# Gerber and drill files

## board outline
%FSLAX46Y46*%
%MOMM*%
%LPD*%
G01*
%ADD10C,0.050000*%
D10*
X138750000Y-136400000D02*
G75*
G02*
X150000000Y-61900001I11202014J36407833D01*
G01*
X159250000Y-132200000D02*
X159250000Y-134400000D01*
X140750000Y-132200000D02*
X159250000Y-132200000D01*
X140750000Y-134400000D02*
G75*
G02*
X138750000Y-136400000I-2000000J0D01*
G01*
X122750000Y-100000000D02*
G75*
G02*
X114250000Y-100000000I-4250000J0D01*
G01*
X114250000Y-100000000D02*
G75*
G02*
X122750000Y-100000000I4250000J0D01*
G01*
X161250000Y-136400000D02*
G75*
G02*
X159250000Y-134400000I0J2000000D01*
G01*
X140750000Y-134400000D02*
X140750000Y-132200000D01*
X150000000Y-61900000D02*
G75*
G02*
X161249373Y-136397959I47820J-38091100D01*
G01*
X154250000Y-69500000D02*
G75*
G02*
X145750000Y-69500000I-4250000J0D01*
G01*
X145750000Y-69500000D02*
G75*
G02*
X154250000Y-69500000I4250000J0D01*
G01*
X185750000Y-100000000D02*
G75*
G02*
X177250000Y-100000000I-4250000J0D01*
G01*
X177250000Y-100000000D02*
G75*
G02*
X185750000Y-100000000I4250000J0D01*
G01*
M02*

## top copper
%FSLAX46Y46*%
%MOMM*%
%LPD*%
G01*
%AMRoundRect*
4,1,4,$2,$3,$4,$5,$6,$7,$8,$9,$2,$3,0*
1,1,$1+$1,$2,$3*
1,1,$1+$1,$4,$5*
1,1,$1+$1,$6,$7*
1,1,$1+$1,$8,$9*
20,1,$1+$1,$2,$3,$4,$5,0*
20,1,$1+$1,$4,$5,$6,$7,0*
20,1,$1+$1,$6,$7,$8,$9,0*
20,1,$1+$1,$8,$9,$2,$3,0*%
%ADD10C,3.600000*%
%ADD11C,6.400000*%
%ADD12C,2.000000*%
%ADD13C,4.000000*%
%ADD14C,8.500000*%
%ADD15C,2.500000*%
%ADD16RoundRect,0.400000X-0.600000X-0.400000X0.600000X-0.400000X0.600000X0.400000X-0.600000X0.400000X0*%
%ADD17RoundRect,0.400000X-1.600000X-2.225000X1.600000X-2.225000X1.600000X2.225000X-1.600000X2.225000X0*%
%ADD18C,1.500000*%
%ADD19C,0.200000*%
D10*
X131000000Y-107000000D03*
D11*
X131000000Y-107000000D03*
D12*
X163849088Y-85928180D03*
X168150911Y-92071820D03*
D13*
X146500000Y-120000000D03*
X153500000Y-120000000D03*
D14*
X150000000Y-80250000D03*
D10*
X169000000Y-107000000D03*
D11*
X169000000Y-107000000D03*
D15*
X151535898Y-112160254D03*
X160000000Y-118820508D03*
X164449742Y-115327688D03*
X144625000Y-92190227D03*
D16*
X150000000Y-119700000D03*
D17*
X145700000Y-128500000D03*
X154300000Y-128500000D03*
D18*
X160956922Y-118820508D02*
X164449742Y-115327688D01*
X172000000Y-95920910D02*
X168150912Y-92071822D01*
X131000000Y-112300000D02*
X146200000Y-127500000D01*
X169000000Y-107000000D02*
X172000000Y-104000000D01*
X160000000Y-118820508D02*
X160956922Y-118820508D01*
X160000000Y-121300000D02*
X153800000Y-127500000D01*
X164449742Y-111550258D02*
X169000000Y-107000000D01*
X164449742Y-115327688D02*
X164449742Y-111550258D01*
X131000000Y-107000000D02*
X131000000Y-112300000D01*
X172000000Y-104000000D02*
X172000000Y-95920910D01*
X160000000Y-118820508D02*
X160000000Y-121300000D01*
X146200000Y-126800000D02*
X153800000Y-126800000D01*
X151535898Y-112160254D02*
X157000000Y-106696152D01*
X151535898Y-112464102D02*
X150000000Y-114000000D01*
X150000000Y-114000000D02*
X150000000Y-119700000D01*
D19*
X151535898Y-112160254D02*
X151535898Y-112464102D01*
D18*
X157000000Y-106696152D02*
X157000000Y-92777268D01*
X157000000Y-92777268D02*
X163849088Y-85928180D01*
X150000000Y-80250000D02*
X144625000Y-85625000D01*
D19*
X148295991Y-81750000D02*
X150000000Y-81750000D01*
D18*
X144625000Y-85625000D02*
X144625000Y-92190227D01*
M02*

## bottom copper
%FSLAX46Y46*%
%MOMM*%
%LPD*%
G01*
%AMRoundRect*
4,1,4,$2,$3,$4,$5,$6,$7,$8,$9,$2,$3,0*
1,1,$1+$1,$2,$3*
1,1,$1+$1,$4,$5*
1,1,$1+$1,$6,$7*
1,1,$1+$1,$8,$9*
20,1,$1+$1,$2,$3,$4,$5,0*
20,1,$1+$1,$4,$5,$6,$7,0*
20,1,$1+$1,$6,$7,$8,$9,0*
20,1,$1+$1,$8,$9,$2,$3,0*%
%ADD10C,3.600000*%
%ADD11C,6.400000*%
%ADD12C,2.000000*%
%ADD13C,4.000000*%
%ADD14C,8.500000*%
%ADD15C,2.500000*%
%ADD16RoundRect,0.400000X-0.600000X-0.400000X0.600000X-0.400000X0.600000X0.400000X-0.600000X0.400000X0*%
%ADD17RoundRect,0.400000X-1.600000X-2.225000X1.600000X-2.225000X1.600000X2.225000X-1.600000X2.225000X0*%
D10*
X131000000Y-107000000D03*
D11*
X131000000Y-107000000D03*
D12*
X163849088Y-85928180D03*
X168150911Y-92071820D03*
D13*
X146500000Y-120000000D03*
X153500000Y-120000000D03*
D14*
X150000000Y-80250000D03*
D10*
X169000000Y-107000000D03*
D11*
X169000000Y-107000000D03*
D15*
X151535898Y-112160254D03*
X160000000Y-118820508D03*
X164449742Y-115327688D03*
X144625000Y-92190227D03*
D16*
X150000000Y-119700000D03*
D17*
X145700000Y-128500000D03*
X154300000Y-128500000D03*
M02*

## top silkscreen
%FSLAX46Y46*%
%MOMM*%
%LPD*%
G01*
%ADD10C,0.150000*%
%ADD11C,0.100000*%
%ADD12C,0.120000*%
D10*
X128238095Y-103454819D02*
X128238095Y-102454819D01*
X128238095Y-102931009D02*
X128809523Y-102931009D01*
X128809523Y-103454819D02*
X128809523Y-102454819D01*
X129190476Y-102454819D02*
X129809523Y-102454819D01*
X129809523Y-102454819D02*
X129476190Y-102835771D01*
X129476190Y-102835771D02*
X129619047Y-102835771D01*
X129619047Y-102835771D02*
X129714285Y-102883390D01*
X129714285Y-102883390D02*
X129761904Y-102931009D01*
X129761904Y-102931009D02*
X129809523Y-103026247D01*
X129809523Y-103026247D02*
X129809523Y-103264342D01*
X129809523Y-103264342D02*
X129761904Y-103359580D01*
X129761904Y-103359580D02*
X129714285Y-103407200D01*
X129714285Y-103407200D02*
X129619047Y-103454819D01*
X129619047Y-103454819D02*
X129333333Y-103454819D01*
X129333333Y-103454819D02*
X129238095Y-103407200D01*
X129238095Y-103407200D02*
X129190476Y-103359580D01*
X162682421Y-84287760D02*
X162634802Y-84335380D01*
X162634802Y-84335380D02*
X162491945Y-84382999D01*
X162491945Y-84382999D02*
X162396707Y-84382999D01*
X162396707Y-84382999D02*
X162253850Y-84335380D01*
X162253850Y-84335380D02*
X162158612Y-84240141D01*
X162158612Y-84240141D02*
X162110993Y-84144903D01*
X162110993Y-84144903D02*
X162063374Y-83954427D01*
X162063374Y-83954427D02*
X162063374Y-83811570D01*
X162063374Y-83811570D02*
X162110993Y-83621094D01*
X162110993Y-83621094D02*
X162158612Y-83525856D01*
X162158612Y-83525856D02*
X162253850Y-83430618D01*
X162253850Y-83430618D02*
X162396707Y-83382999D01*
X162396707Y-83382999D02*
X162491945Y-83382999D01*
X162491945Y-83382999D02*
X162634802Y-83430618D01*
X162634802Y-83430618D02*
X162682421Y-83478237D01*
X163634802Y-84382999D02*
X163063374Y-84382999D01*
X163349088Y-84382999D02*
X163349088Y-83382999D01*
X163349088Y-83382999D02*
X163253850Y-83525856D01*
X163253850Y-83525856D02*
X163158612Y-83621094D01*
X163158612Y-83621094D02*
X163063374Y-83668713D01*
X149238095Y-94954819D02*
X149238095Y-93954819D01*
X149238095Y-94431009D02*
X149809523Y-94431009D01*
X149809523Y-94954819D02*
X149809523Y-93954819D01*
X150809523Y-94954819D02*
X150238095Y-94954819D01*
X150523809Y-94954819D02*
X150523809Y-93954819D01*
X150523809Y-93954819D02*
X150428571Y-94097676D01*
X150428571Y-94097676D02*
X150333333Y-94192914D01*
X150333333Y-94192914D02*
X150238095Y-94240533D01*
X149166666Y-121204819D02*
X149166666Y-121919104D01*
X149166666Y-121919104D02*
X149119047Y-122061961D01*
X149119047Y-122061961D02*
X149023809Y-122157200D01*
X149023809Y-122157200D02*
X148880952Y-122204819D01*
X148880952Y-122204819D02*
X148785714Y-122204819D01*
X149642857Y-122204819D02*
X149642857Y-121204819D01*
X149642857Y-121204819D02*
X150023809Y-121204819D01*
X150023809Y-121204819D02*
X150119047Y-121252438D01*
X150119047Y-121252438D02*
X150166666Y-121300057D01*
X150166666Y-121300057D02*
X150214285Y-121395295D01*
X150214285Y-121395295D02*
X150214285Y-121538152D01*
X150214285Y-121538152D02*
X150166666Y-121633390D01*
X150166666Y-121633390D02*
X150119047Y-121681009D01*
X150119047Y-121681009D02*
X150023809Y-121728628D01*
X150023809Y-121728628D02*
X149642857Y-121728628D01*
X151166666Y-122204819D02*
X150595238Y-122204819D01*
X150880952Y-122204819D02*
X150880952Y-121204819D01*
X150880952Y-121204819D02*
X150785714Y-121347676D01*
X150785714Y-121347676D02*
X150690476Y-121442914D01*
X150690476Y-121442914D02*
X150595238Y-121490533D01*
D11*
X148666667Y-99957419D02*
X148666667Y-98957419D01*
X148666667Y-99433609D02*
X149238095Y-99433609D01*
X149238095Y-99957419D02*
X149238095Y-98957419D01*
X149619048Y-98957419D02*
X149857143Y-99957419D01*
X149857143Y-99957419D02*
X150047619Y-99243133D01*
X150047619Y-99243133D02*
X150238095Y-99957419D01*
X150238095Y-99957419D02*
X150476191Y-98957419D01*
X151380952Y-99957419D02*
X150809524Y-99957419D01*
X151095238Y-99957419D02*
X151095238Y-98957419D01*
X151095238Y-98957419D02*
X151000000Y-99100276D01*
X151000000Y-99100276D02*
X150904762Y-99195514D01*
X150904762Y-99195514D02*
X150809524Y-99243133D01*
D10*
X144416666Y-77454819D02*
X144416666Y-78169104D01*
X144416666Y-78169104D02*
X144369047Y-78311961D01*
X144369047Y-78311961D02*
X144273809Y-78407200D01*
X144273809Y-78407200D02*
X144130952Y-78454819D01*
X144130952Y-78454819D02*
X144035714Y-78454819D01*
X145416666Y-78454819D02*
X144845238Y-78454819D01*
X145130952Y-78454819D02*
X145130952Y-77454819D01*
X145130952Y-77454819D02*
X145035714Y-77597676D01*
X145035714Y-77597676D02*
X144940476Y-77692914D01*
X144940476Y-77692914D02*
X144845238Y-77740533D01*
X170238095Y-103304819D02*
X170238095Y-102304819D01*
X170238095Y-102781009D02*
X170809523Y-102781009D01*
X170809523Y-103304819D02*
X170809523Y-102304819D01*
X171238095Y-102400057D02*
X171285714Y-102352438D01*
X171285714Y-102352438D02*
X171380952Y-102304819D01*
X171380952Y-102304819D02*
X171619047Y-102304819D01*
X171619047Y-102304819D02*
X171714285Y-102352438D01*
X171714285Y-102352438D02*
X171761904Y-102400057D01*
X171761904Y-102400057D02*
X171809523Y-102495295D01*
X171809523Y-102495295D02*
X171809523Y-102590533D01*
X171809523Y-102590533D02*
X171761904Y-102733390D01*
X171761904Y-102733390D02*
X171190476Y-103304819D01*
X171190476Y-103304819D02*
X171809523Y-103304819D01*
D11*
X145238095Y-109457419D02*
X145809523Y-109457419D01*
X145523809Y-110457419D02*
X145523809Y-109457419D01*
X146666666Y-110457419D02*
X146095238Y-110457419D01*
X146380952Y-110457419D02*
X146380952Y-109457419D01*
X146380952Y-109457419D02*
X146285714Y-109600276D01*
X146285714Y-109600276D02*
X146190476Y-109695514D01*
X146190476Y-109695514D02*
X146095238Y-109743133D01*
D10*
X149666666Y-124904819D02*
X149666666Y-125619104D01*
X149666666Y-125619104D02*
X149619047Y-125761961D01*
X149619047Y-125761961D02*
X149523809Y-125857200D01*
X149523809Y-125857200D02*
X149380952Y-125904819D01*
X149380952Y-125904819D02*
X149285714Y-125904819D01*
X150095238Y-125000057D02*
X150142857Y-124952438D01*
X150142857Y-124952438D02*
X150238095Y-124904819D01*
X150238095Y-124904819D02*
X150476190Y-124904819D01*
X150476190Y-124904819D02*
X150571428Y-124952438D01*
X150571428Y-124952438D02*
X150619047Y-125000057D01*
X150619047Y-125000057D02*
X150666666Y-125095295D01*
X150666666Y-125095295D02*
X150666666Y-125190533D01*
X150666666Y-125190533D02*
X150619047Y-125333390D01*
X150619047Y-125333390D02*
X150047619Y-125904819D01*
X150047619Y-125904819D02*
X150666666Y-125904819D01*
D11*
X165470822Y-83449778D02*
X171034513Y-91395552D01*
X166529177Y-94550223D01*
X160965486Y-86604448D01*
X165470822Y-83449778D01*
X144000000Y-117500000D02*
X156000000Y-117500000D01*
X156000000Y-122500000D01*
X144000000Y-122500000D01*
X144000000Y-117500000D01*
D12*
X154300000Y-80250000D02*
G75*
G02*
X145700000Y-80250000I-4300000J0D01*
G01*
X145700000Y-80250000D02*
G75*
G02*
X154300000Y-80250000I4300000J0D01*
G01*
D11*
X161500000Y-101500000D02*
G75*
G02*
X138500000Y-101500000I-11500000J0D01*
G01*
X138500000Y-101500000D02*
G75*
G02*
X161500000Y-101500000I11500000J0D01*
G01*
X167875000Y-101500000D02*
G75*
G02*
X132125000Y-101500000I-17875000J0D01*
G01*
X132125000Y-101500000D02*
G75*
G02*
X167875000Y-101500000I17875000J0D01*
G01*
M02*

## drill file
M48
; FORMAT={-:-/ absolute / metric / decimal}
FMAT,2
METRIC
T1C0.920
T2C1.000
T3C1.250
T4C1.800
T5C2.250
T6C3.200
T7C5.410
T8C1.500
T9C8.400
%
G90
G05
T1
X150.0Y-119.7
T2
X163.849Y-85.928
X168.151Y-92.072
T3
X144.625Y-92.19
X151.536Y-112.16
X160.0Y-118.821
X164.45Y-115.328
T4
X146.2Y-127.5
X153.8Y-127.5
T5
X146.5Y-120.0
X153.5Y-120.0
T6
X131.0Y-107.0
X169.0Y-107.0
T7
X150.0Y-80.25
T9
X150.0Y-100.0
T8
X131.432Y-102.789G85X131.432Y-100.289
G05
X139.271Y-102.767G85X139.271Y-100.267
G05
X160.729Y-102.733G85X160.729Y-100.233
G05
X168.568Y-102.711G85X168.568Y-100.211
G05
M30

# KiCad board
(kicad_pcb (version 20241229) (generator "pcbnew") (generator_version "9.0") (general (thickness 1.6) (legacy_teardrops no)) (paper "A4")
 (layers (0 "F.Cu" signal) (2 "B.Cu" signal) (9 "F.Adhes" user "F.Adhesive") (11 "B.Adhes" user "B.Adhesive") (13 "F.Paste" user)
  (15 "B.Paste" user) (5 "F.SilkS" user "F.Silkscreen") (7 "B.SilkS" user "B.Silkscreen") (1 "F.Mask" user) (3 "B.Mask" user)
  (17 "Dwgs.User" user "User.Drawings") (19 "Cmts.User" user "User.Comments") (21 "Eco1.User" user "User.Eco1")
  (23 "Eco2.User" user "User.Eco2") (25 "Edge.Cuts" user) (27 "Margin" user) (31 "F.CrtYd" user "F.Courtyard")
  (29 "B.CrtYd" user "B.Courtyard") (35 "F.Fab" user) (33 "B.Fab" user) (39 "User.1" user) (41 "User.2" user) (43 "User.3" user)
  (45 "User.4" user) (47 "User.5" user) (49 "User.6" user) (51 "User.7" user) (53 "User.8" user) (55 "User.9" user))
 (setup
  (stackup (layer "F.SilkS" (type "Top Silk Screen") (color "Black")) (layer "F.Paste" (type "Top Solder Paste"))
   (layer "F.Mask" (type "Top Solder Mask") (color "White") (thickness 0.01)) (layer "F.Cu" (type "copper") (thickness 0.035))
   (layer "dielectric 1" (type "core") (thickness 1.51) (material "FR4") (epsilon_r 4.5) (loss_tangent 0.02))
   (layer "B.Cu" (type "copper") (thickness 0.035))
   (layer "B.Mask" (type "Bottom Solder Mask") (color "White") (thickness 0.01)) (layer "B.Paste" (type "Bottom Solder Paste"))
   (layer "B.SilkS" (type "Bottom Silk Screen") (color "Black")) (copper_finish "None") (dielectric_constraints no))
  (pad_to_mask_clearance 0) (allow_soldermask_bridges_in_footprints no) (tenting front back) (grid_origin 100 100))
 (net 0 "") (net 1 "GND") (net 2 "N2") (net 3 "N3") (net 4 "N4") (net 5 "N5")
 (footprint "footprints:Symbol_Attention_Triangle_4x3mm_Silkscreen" (layer "F.Cu") (at 175 111.5)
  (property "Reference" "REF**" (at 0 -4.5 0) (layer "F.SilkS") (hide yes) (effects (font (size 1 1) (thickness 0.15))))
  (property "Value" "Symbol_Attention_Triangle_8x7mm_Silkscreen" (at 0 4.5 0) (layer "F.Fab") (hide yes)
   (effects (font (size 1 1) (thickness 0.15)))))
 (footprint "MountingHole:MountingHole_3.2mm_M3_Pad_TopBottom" (layer "F.Cu") (at 131 107)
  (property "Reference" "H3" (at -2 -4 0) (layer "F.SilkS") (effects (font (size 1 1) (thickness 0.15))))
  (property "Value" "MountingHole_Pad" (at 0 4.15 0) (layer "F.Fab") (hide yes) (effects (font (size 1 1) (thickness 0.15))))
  (pad "1" thru_hole circle (at 0 0) (size 3.6 3.6) (drill 3.2) (layers "*.Cu" "*.Mask") (remove_unused_layers no) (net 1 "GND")
   (zone_connect 2))
  (pad "1" connect circle (at 0 0) (size 6.4 6.4) (layers "F.Cu" "F.Mask") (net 1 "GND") (zone_connect 2))
  (pad "1" connect circle (at 0 0) (size 6.4 6.4) (layers "B.Cu" "B.Mask") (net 1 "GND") (zone_connect 2)))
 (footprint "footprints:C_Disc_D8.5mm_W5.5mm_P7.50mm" (layer "F.Cu") (at 163.849088 85.92818 -55)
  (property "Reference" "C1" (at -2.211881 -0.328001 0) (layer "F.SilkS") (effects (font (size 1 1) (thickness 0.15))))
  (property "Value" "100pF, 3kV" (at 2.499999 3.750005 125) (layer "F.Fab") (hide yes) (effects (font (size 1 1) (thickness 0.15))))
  (fp_poly
   (pts (xy -1.1 -2.75) (xy 8.599999 -2.75) (xy 8.6 2.75) (xy -1.1 2.75)) (stroke (width 0.1) (type solid)) (fill no) (layer "F.SilkS"))
  (pad "1" thru_hole circle (at 0 0 305) (size 2 2) (drill 1) (layers "*.Cu" "*.Mask") (remove_unused_layers no) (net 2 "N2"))
  (pad "2" thru_hole circle (at 7.5 0 305) (size 2 2) (drill 1) (layers "*.Cu" "*.Mask") (remove_unused_layers no) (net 1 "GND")))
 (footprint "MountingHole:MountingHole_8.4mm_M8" (layer "F.Cu") (at 150 100)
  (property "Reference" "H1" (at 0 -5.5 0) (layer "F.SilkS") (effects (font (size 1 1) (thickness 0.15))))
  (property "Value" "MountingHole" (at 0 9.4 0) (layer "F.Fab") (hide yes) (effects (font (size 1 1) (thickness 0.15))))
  (pad "" np_thru_hole circle (at 0 0) (size 8.4 8.4) (drill 8.4) (layers "*.Cu" "*.Mask")))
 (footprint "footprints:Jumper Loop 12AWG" (layer "F.Cu") (at 146.5 120)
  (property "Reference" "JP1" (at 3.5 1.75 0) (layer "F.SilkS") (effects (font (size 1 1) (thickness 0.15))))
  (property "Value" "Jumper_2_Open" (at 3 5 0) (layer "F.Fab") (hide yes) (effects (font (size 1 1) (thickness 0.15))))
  (fp_rect (start -2.5 -2.5) (end 9.5 2.5) (stroke (width 0.1) (type solid)) (fill no) (layer "F.SilkS"))
  (pad "1" thru_hole circle (at 0 0) (size 4 4) (drill 2.25) (layers "*.Cu" "*.Mask") (remove_unused_layers no) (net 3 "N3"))
  (pad "2" thru_hole circle (at 7 0) (size 4 4) (drill 2.25) (layers "*.Cu" "*.Mask") (remove_unused_layers no) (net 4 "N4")))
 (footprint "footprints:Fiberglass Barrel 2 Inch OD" (layer "F.Cu") (at 150 100)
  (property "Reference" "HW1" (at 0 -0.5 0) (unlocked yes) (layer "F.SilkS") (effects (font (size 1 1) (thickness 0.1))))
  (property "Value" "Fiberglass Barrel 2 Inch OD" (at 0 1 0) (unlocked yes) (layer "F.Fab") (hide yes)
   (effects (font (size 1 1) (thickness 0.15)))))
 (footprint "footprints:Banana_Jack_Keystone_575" (layer "F.Cu") (at 150 80.25)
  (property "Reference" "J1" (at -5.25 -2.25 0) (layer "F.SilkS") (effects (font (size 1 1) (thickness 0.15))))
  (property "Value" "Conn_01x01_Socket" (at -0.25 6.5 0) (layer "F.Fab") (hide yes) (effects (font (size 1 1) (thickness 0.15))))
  (fp_circle (center 0 0) (end 4.3 0) (stroke (width 0.12) (type solid)) (fill no) (layer "F.SilkS"))
  (pad "1" thru_hole circle (at 0 0) (size 8.5 8.5) (drill 5.41) (layers "*.Cu" "*.Mask") (remove_unused_layers no) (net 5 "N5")))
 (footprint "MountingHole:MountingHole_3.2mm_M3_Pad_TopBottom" (layer "F.Cu") (at 169 107)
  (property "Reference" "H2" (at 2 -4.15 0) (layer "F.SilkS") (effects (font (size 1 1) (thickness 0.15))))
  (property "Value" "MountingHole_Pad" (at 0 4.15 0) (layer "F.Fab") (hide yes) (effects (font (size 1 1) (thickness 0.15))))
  (pad "1" thru_hole circle (at 0 0) (size 3.6 3.6) (drill 3.2) (layers "*.Cu" "*.Mask") (remove_unused_layers no) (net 1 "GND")
   (zone_connect 2))
  (pad "1" connect circle (at 0 0) (size 6.4 6.4) (layers "F.Cu" "F.Mask") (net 1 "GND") (zone_connect 2))
  (pad "1" connect circle (at 0 0) (size 6.4 6.4) (layers "B.Cu" "B.Mask") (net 1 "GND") (zone_connect 2)))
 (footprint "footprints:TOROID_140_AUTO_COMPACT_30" (layer "F.Cu") (at 150 101.5 30)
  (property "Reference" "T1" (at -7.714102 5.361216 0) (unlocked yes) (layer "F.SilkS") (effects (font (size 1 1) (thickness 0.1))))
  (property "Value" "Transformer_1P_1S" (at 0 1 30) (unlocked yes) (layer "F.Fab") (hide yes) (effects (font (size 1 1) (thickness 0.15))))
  (fp_circle (center 0 0) (end 11.5 0) (stroke (width 0.1) (type default)) (fill no) (layer "F.SilkS"))
  (fp_circle (center 0 0) (end 17.875 0) (stroke (width 0.1) (type default)) (fill no) (layer "F.SilkS"))
  (pad "" np_thru_hole rect (at -16.1 -9.25 90) (size 5 3) (drill oval 4 1.5) (layers))
  (pad "" np_thru_hole rect (at -9.3 -5.35 90) (size 5 3) (drill oval 4 1.5) (layers))
  (pad "" np_thru_hole rect (at 9.3 5.35 90) (size 5 3) (drill oval 4 1.5) (layers))
  (pad "" np_thru_hole rect (at 16.1 9.25 90) (size 5 3) (drill oval 4 1.5) (layers))
  (pad "1" thru_hole circle (at -4 10 30) (size 2.5 2.5) (drill 1.25) (layers "*.Cu" "*.Mask") (remove_unused_layers no) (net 2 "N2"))
  (pad "2" thru_hole circle (at 0 20 30) (size 2.5 2.5) (drill 1.25) (layers "*.Cu" "*.Mask") (remove_unused_layers no) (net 1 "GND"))
  (pad "3" thru_hole circle (at 5.6 19.2 30) (size 2.5 2.5) (drill 1.25) (layers "*.Cu" "*.Mask") (remove_unused_layers no) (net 1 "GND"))
  (pad "4" thru_hole circle (at 0 -10.75 30) (size 2.5 2.5) (drill 1.25) (layers "*.Cu" "*.Mask") (remove_unused_layers no) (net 5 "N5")))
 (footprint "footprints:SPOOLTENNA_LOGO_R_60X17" (layer "B.Cu") (at 150 89 180)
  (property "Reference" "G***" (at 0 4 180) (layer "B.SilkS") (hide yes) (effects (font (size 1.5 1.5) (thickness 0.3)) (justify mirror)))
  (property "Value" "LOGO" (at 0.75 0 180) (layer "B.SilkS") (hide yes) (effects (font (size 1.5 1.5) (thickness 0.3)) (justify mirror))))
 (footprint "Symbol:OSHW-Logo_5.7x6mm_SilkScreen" (layer "B.Cu") (at 166 127 180)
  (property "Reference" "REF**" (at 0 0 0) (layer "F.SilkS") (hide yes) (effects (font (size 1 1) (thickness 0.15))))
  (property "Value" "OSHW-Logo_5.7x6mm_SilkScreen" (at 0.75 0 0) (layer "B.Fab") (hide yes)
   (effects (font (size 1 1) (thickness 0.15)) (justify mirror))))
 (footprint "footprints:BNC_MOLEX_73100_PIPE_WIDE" (layer "B.Cu") (at 150 119.7)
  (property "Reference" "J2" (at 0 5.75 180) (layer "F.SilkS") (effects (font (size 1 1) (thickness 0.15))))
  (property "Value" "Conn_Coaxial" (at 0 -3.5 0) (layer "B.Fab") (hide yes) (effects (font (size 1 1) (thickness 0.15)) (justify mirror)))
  (pad "1" thru_hole roundrect (at 0 0) (size 2 1.6) (drill 0.92) (layers "*.Cu" "*.Mask") (remove_unused_layers no) (roundrect_rratio 0.25)
   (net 2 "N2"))
  (pad "2" thru_hole roundrect (at -3.8 7.8) (size 4 5.25) (drill 1.8 (offset -0.5 1)) (layers "*.Cu" "*.Mask") (remove_unused_layers no)
   (roundrect_rratio 0.1) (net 1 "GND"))
  (pad "2" thru_hole roundrect (at 3.8 7.8) (size 4 5.25) (drill 1.8 (offset 0.5 1)) (layers "*.Cu" "*.Mask") (remove_unused_layers no)
   (roundrect_rratio 0.1) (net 1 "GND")))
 (gr_arc (start 138.75 136.4) (mid 112.286837 94.304471) (end 150 61.9) (stroke (width 0.05) (type default)) (layer "Edge.Cuts"))
 (gr_line (start 159.25 132.2) (end 159.25 134.4) (stroke (width 0.05) (type solid)) (layer "Edge.Cuts"))
 (gr_line (start 140.75 132.2) (end 159.25 132.2) (stroke (width 0.05) (type solid)) (layer "Edge.Cuts"))
 (gr_arc (start 140.75 134.4) (mid 140.164214 135.814214) (end 138.75 136.4) (stroke (width 0.05) (type default)) (layer "Edge.Cuts"))
 (gr_circle (center 118.5 100) (end 122.75 100) (stroke (width 0.05) (type solid)) (fill no) (layer "Edge.Cuts"))
 (gr_arc (start 161.25 136.4) (mid 159.835785 135.814214) (end 159.25 134.4) (stroke (width 0.05) (type default)) (layer "Edge.Cuts"))
 (gr_line (start 140.75 134.4) (end 140.75 132.2) (stroke (width 0.05) (type solid)) (layer "Edge.Cuts"))
 (gr_arc (start 150 61.9) (mid 187.711966 94.30372) (end 161.249371 136.397954) (stroke (width 0.05) (type default)) (layer "Edge.Cuts"))
 (gr_circle (center 150 69.5) (end 154.25 69.5) (stroke (width 0.05) (type solid)) (fill no) (layer "Edge.Cuts"))
 (gr_circle (center 181.5 100) (end 185.75 100) (stroke (width 0.05) (type solid)) (fill no) (layer "Edge.Cuts"))
 (segment (start 160.956922 118.820508) (end 164.449742 115.327688) (width 1.5) (layer "F.Cu") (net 1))
 (segment (start 172 95.92091) (end 168.150912 92.071822) (width 1.5) (layer "F.Cu") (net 1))
 (segment (start 131 112.3) (end 146.2 127.5) (width 1.5) (layer "F.Cu") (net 1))
 (segment (start 169 107) (end 172 104) (width 1.5) (layer "F.Cu") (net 1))
 (segment (start 160 118.820508) (end 160.956922 118.820508) (width 1.5) (layer "F.Cu") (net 1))
 (segment (start 160 121.3) (end 153.8 127.5) (width 1.5) (layer "F.Cu") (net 1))
 (segment (start 164.449742 111.550258) (end 169 107) (width 1.5) (layer "F.Cu") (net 1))
 (segment (start 164.449742 115.327688) (end 164.449742 111.550258) (width 1.5) (layer "F.Cu") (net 1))
 (segment (start 131 107) (end 131 112.3) (width 1.5) (layer "F.Cu") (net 1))
 (segment (start 172 104) (end 172 95.92091) (width 1.5) (layer "F.Cu") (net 1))
 (segment (start 160 118.820508) (end 160 121.3) (width 1.5) (layer "F.Cu") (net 1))
 (segment (start 146.2 126.8) (end 153.8 126.8) (width 1.5) (layer "F.Cu") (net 1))
 (segment (start 151.535898 112.160254) (end 157 106.696152) (width 1.5) (layer "F.Cu") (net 2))
 (segment (start 151.535898 112.464102) (end 150 114) (width 1.5) (layer "F.Cu") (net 2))
 (segment (start 150 114) (end 150 119.7) (width 1.5) (layer "F.Cu") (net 2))
 (segment (start 151.535898 112.160254) (end 151.535898 112.464102) (width 0.2) (layer "F.Cu") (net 2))
 (segment (start 157 106.696152) (end 157 92.777268) (width 1.5) (layer "F.Cu") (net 2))
 (segment (start 157 92.777268) (end 163.849088 85.92818) (width 1.5) (layer "F.Cu") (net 2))
 (segment (start 150 80.25) (end 144.625 85.625) (width 1.5) (layer "F.Cu") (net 5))
 (segment (start 148.295991 81.75) (end 150 81.75) (width 0.2) (layer "F.Cu") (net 5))
 (segment (start 144.625 85.625) (end 144.625 92.190227) (width 1.5) (layer "F.Cu") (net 5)))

